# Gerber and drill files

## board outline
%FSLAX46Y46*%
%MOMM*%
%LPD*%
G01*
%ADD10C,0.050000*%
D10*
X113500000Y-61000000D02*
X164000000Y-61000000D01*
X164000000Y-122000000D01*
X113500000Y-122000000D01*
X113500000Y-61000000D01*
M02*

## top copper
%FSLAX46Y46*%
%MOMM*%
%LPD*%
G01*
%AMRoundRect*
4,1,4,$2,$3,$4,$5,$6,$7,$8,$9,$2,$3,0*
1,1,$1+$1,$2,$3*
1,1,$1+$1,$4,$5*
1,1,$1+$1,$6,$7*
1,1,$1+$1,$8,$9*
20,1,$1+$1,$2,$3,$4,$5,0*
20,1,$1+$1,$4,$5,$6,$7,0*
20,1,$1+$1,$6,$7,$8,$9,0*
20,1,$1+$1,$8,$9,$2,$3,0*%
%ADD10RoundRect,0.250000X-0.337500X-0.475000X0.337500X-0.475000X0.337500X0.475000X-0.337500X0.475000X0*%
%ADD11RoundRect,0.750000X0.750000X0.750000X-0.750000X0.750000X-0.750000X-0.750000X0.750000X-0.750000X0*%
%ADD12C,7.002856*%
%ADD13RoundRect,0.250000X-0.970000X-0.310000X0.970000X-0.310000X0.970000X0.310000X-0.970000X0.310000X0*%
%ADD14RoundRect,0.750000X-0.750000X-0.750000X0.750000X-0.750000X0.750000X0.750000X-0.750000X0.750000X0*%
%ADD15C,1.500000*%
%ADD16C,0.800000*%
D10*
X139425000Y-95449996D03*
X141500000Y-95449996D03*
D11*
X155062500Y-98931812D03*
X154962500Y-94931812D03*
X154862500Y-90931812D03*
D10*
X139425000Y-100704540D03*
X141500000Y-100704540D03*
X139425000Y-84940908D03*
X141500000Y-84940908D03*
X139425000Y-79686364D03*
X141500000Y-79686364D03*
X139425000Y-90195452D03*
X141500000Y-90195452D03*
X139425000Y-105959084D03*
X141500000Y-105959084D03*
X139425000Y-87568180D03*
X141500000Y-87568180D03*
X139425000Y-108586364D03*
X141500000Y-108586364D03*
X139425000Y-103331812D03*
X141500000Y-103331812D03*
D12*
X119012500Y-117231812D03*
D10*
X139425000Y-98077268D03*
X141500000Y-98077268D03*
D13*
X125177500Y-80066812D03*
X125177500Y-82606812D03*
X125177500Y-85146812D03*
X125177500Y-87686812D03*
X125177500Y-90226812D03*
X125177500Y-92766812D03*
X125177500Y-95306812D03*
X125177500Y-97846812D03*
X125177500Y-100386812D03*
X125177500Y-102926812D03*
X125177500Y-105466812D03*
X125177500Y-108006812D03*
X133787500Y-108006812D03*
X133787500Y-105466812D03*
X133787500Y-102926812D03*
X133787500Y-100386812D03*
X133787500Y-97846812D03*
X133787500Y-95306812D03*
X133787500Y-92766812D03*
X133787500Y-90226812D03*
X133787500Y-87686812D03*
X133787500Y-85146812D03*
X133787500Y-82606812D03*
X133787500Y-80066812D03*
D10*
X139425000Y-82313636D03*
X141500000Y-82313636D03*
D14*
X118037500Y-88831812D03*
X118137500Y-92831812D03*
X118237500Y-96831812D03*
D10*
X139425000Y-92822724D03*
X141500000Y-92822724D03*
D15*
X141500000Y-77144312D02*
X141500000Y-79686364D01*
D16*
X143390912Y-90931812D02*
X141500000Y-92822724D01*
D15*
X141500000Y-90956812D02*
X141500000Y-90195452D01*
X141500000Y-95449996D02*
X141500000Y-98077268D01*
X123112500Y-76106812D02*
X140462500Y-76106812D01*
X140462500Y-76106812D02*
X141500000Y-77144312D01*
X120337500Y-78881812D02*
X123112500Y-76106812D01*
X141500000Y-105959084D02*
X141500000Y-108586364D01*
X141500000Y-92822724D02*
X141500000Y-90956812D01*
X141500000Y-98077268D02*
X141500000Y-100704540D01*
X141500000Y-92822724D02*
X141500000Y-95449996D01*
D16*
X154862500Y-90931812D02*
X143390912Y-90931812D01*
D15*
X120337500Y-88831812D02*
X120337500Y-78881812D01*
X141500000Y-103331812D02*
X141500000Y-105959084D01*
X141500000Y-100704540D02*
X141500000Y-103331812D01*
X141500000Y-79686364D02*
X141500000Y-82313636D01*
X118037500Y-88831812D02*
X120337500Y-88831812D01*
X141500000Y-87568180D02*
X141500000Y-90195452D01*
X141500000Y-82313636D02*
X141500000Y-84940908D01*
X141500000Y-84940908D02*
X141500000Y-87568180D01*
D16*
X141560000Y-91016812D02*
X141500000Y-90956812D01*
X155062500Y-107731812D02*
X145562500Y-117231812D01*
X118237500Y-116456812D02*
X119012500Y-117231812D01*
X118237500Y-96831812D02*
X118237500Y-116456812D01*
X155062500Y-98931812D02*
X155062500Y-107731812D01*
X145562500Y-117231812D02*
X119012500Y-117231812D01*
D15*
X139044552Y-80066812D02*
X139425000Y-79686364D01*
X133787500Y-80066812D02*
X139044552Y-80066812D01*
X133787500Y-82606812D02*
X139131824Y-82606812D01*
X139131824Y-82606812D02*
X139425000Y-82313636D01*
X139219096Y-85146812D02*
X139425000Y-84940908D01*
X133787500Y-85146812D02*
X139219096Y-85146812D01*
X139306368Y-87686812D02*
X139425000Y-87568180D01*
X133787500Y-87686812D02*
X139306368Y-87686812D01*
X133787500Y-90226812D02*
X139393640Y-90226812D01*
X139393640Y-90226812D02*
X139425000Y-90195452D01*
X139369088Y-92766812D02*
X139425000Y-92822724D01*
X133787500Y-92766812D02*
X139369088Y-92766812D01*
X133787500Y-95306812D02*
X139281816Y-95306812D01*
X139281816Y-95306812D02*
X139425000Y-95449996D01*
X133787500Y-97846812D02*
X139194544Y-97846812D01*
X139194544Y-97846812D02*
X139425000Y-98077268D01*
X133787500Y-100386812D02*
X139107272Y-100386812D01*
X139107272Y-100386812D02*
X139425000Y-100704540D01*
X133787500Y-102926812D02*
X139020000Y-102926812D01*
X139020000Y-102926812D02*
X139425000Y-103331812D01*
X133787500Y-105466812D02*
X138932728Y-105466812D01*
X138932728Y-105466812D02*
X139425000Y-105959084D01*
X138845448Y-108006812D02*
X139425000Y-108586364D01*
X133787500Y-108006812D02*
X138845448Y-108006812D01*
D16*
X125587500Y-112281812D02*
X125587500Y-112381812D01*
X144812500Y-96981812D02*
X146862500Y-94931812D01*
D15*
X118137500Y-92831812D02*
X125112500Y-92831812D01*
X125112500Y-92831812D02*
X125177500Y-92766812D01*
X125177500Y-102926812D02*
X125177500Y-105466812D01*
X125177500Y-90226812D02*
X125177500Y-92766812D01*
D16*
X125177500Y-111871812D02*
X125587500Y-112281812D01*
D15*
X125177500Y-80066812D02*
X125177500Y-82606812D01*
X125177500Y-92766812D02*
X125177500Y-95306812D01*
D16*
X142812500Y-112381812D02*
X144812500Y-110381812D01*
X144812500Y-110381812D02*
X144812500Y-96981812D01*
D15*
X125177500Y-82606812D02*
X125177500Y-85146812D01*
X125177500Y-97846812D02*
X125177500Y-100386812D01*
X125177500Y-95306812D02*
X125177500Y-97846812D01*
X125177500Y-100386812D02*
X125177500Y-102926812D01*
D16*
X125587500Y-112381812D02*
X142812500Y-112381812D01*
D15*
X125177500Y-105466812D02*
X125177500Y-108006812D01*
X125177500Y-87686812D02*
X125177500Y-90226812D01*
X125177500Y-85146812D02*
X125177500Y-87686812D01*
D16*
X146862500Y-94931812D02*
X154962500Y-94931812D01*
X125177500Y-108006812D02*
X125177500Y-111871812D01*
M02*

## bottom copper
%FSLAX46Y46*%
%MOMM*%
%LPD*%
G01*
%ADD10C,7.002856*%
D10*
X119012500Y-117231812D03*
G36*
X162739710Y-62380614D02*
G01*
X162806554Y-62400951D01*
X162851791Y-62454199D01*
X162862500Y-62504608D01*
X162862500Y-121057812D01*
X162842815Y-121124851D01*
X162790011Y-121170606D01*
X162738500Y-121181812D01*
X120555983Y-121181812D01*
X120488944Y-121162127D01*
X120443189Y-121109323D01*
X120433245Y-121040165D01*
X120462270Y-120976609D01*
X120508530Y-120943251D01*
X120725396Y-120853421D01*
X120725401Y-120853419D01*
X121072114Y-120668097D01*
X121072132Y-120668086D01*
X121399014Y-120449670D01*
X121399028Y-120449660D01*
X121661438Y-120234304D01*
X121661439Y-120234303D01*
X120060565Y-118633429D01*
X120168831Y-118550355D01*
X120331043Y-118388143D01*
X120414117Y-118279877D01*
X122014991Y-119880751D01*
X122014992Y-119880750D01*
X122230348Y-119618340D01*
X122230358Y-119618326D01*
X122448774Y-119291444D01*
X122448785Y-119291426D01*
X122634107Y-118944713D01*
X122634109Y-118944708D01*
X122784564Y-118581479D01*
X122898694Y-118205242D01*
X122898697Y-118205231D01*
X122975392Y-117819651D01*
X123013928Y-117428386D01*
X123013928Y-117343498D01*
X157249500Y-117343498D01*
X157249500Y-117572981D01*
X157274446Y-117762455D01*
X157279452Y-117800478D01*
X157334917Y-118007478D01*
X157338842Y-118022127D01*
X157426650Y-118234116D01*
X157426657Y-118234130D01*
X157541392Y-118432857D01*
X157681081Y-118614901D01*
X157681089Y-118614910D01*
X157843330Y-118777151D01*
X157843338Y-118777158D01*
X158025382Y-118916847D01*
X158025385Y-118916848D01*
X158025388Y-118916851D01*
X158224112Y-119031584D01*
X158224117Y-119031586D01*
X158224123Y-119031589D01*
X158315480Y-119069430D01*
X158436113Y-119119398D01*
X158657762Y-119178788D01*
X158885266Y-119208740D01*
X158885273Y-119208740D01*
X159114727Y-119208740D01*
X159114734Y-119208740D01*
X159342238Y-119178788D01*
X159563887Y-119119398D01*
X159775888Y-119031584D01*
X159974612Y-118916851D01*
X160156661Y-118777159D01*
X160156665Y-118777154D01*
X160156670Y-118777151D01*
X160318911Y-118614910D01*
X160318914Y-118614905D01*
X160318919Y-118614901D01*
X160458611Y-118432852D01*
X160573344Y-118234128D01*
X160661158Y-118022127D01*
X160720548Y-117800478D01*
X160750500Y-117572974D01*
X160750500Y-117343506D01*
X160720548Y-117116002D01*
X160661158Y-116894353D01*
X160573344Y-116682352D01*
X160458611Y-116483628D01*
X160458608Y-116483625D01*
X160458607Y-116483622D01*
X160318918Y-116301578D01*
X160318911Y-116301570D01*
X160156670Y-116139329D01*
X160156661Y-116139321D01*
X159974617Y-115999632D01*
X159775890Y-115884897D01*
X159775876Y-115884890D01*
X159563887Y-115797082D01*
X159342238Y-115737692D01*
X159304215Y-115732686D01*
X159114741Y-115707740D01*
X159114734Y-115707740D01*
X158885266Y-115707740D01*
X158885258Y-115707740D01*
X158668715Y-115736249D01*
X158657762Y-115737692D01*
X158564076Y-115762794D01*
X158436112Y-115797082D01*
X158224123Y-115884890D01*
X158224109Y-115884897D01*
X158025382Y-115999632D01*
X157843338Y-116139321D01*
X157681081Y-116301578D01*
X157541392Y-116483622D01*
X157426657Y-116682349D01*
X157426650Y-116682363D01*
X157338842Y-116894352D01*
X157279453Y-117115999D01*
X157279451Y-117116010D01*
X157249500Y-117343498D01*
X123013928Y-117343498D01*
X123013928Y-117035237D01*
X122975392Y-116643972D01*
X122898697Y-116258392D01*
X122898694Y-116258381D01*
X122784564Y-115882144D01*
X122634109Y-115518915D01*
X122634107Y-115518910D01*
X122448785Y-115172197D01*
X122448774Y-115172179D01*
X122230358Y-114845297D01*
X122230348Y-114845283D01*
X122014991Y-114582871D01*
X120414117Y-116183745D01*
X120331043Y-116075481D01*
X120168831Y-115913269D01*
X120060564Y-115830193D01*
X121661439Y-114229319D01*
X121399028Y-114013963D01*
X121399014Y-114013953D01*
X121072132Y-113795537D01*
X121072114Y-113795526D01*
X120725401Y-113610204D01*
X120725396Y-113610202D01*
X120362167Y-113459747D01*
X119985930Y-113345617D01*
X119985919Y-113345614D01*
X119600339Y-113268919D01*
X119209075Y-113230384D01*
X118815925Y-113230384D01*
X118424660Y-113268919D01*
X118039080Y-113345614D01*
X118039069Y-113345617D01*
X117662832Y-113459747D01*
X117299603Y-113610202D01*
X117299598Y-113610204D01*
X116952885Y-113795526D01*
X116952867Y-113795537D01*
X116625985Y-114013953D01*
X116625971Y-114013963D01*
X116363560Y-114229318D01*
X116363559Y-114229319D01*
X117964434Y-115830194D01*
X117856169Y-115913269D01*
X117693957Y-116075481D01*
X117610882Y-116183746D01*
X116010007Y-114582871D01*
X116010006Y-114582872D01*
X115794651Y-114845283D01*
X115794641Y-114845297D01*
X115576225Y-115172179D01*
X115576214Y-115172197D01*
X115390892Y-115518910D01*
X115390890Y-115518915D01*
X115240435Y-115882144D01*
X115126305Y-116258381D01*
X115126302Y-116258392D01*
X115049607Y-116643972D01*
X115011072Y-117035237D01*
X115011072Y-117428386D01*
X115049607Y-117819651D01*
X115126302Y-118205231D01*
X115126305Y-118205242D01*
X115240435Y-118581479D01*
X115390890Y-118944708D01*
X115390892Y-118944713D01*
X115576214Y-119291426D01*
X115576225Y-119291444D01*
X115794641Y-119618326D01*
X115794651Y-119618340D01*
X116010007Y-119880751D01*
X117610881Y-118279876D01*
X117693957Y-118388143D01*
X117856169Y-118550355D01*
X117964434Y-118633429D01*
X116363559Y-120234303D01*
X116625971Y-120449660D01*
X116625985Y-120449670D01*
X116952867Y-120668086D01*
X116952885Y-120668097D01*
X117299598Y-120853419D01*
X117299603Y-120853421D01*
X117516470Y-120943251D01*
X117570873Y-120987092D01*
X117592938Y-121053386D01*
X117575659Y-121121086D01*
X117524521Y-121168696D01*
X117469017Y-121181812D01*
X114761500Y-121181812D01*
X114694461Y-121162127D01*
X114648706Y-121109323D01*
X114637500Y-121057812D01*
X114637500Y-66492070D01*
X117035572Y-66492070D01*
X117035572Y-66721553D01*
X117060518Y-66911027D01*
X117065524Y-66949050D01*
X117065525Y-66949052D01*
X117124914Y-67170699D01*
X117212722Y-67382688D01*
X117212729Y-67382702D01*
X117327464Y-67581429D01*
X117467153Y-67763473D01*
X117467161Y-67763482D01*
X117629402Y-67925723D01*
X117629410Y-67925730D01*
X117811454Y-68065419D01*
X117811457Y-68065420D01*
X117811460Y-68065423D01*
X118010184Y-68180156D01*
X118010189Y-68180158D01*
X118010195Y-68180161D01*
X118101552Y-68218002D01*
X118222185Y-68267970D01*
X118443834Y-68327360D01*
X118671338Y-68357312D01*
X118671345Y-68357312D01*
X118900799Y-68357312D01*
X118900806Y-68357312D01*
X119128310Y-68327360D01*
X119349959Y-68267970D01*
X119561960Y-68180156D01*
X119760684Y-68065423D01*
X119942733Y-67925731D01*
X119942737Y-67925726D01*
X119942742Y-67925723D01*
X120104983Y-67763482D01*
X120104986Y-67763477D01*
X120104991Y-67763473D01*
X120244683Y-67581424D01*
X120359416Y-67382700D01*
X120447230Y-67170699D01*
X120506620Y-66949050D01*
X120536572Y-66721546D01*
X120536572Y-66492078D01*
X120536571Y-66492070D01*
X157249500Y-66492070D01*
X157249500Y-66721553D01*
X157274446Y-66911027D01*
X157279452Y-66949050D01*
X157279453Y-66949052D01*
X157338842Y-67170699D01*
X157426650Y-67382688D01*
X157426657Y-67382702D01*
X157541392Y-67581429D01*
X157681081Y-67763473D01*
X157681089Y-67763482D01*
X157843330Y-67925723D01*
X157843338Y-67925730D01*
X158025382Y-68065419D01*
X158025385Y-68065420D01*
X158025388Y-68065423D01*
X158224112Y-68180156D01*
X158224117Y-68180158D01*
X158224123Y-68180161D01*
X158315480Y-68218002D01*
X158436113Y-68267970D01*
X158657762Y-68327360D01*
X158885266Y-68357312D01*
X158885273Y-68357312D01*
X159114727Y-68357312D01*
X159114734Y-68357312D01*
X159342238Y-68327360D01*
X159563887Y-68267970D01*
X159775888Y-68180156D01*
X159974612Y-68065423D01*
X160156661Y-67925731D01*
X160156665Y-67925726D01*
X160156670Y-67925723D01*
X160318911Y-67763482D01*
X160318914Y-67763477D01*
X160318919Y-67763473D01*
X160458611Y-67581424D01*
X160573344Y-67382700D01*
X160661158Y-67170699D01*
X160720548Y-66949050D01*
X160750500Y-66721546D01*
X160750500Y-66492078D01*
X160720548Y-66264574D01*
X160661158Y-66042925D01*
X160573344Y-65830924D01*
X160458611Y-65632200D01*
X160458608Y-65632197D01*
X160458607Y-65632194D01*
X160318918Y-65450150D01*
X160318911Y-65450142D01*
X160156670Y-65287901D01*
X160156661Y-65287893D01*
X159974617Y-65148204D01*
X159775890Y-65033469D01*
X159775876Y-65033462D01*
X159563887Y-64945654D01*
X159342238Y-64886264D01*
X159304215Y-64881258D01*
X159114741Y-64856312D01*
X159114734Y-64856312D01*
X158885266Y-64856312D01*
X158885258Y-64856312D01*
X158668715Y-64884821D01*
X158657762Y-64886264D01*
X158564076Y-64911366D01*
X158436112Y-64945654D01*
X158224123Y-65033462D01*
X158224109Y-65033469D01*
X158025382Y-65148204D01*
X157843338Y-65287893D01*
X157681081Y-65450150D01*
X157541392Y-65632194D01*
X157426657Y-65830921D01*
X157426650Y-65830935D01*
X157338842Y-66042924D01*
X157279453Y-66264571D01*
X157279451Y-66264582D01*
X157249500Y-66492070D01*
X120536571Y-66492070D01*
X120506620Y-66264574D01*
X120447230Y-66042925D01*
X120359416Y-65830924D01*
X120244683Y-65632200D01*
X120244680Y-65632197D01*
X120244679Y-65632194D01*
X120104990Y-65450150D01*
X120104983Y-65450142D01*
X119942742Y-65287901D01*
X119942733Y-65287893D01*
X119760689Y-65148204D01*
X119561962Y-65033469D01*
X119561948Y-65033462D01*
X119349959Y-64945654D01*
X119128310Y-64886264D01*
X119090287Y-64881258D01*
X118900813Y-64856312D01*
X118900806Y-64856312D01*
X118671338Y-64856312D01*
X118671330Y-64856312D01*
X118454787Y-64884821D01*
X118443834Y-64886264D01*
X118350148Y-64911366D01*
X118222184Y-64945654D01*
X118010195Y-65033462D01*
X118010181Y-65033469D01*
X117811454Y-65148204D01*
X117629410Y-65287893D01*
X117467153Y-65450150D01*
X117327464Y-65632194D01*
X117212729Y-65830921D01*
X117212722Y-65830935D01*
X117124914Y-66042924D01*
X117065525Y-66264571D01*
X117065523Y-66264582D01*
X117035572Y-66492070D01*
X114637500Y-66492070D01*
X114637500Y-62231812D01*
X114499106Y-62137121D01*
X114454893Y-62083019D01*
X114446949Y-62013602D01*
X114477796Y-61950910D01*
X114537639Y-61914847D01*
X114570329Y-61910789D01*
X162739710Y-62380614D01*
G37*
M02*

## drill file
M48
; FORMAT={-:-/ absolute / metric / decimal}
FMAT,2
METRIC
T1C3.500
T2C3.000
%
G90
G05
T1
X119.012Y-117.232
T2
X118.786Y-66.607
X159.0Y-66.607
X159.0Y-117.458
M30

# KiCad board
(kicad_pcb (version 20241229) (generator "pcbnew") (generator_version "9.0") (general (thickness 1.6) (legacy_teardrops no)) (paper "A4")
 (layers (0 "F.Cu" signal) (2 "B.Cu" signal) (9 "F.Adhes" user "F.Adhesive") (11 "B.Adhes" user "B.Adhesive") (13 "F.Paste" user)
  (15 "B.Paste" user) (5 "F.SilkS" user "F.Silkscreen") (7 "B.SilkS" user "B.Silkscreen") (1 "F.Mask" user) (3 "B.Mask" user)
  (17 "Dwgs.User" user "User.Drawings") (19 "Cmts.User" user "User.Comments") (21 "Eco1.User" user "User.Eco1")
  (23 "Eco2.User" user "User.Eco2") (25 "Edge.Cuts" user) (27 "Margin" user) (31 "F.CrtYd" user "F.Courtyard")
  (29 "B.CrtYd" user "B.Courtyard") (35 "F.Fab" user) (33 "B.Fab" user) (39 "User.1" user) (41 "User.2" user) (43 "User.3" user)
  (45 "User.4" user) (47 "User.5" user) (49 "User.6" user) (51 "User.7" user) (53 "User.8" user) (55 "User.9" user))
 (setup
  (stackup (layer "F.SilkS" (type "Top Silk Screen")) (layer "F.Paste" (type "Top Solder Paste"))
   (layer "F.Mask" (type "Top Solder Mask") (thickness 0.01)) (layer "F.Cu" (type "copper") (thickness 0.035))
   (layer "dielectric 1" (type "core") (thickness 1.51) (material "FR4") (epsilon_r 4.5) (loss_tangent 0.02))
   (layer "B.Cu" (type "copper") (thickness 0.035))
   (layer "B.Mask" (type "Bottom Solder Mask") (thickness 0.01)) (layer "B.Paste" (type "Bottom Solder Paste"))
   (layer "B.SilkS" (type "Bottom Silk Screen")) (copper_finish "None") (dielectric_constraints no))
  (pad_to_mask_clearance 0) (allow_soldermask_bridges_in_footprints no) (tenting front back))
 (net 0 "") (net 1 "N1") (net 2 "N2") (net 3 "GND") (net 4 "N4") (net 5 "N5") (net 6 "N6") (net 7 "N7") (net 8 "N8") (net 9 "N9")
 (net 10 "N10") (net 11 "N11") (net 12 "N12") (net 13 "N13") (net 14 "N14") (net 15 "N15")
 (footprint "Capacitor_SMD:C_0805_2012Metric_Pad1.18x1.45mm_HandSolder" (layer "F.Cu") (at 140.4625 95.449996)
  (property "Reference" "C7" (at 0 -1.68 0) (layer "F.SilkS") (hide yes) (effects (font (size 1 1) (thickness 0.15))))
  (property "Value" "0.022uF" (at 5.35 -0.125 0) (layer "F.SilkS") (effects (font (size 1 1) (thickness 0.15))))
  (pad "1" smd roundrect (at -1.0375 0) (size 1.175 1.45) (layers "F.Cu" "F.Mask" "F.Paste") (roundrect_rratio 0.212766) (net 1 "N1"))
  (pad "2" smd roundrect (at 1.0375 0) (size 1.175 1.45) (layers "F.Cu" "F.Mask" "F.Paste") (roundrect_rratio 0.212766) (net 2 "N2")))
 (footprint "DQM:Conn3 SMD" (layer "F.Cu") (at 155.0625 95.031812 180)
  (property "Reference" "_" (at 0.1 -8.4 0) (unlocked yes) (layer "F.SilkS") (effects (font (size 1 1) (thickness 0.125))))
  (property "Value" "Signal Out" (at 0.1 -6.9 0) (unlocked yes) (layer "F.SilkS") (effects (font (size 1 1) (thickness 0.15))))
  (pad "1" smd roundrect (at 0 -3.9 180) (size 3 3) (layers "F.Cu" "F.Mask" "F.Paste") (roundrect_rratio 0.25) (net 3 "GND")
   (thermal_bridge_angle 45))
  (pad "2" smd roundrect (at 0.1 0.1 180) (size 3 3) (layers "F.Cu" "F.Mask" "F.Paste") (roundrect_rratio 0.25) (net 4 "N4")
   (thermal_bridge_angle 45))
  (pad "3" smd roundrect (at 0.2 4.1 180) (size 3 3) (layers "F.Cu" "F.Mask" "F.Paste") (roundrect_rratio 0.25) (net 2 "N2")
   (thermal_bridge_angle 45)))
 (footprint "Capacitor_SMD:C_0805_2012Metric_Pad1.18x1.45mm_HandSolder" (layer "F.Cu") (at 140.4625 100.70454)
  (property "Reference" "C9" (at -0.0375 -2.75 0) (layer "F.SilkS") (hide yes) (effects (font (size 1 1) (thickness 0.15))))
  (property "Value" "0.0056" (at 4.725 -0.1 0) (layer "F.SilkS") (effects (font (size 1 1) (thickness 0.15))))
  (pad "1" smd roundrect (at -1.0375 0) (size 1.175 1.45) (layers "F.Cu" "F.Mask" "F.Paste") (roundrect_rratio 0.212766) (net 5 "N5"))
  (pad "2" smd roundrect (at 1.0375 0) (size 1.175 1.45) (layers "F.Cu" "F.Mask" "F.Paste") (roundrect_rratio 0.212766) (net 2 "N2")))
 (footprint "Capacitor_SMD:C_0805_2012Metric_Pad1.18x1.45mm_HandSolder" (layer "F.Cu") (at 140.4625 84.940908)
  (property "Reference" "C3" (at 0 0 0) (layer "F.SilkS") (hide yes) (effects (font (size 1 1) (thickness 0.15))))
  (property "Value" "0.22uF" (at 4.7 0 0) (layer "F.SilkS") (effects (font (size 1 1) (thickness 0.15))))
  (pad "1" smd roundrect (at -1.0375 0) (size 1.175 1.45) (layers "F.Cu" "F.Mask" "F.Paste") (roundrect_rratio 0.212766) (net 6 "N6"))
  (pad "2" smd roundrect (at 1.0375 0) (size 1.175 1.45) (layers "F.Cu" "F.Mask" "F.Paste") (roundrect_rratio 0.212766) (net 2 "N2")))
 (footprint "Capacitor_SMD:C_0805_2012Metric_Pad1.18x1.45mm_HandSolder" (layer "F.Cu") (at 140.4625 79.686364)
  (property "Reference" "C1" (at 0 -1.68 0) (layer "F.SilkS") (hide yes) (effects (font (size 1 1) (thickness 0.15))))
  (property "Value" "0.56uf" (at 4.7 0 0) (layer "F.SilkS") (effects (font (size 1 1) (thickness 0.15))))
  (pad "1" smd roundrect (at -1.0375 0) (size 1.175 1.45) (layers "F.Cu" "F.Mask" "F.Paste") (roundrect_rratio 0.212766) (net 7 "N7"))
  (pad "2" smd roundrect (at 1.0375 0) (size 1.175 1.45) (layers "F.Cu" "F.Mask" "F.Paste") (roundrect_rratio 0.212766) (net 2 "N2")))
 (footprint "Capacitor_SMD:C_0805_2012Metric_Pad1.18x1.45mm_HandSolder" (layer "F.Cu") (at 140.4625 90.195452)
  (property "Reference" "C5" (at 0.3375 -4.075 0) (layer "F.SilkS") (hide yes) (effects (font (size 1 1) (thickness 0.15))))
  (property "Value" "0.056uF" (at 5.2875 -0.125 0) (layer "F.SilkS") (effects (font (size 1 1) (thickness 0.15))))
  (pad "1" smd roundrect (at -1.0375 0) (size 1.175 1.45) (layers "F.Cu" "F.Mask" "F.Paste") (roundrect_rratio 0.212766) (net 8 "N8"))
  (pad "2" smd roundrect (at 1.0375 0) (size 1.175 1.45) (layers "F.Cu" "F.Mask" "F.Paste") (roundrect_rratio 0.212766) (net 2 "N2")))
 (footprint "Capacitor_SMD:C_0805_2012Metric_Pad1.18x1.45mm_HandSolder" (layer "F.Cu") (at 140.4625 105.959084)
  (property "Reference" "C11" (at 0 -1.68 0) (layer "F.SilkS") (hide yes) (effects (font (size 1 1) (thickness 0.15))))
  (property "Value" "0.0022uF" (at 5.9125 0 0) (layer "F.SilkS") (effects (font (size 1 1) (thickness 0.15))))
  (pad "1" smd roundrect (at -1.0375 0) (size 1.175 1.45) (layers "F.Cu" "F.Mask" "F.Paste") (roundrect_rratio 0.212766) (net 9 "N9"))
  (pad "2" smd roundrect (at 1.0375 0) (size 1.175 1.45) (layers "F.Cu" "F.Mask" "F.Paste") (roundrect_rratio 0.212766) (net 2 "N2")))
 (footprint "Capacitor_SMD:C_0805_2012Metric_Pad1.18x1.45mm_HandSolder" (layer "F.Cu") (at 140.4625 87.56818)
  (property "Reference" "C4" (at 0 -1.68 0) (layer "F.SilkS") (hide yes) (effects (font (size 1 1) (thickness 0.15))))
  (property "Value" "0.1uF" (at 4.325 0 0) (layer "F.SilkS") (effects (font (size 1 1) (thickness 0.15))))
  (pad "1" smd roundrect (at -1.0375 0) (size 1.175 1.45) (layers "F.Cu" "F.Mask" "F.Paste") (roundrect_rratio 0.212766) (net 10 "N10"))
  (pad "2" smd roundrect (at 1.0375 0) (size 1.175 1.45) (layers "F.Cu" "F.Mask" "F.Paste") (roundrect_rratio 0.212766) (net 2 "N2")))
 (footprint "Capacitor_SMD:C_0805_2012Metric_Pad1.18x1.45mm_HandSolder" (layer "F.Cu") (at 140.4625 108.586364)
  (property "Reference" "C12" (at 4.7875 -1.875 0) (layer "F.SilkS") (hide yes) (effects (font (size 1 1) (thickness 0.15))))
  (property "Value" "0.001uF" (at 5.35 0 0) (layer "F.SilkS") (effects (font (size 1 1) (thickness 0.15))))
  (pad "1" smd roundrect (at -1.0375 0) (size 1.175 1.45) (layers "F.Cu" "F.Mask" "F.Paste") (roundrect_rratio 0.212766) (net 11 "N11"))
  (pad "2" smd roundrect (at 1.0375 0) (size 1.175 1.45) (layers "F.Cu" "F.Mask" "F.Paste") (roundrect_rratio 0.212766) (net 2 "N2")))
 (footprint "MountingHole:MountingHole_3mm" (layer "F.Cu") (at 118.786072 66.606812)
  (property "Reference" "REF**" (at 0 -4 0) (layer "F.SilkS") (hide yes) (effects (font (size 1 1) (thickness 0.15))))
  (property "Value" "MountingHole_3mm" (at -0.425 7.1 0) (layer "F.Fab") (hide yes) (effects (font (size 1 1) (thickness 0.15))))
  (pad "" np_thru_hole circle (at 0 0) (size 3 3) (drill 3) (layers "*.Cu" "*.Mask")))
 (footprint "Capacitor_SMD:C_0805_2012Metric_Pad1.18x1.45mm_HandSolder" (layer "F.Cu") (at 140.4625 103.331812)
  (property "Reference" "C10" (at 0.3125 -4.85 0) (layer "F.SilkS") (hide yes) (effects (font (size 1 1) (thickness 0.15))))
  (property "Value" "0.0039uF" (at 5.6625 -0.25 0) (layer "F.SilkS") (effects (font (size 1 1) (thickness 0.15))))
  (pad "1" smd roundrect (at -1.0375 0) (size 1.175 1.45) (layers "F.Cu" "F.Mask" "F.Paste") (roundrect_rratio 0.212766) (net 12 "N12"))
  (pad "2" smd roundrect (at 1.0375 0) (size 1.175 1.45) (layers "F.Cu" "F.Mask" "F.Paste") (roundrect_rratio 0.212766) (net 2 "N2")))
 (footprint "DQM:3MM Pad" (layer "F.Cu") (at 119.0125 117.231812)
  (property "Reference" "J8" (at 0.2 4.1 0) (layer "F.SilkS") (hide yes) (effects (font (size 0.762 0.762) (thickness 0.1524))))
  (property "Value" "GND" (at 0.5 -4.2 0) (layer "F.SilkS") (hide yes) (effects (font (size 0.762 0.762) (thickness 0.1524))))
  (pad "1" thru_hole circle (at 0 0) (size 7.002856 7.002856) (drill 3.5) (layers "*.Cu" "*.Mask") (remove_unused_layers no) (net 3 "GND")))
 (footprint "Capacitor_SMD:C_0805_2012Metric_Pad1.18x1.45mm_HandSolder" (layer "F.Cu") (at 140.4625 98.077268)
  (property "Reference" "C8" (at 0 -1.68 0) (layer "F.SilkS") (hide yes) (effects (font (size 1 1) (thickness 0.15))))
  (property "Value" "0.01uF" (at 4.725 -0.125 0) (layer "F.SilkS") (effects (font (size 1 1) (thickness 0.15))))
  (pad "1" smd roundrect (at -1.0375 0) (size 1.175 1.45) (layers "F.Cu" "F.Mask" "F.Paste") (roundrect_rratio 0.212766) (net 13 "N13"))
  (pad "2" smd roundrect (at 1.0375 0) (size 1.175 1.45) (layers "F.Cu" "F.Mask" "F.Paste") (roundrect_rratio 0.212766) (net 2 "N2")))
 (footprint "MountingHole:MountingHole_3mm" (layer "F.Cu") (at 159 117.45824)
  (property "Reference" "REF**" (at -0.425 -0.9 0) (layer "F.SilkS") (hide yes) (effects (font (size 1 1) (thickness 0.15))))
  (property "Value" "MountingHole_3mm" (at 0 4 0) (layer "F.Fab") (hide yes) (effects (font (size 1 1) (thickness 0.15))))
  (pad "" np_thru_hole circle (at 0 0) (size 3 3) (drill 3) (layers "*.Cu" "*.Mask")))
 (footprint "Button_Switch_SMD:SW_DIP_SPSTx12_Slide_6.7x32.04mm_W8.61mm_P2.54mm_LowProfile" (layer "F.Cu") (at 129.4825 94.036812)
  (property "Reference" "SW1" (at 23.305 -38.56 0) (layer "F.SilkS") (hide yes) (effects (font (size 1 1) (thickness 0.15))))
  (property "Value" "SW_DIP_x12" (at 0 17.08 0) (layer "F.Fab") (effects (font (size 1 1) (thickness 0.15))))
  (pad "1" smd roundrect (at -4.305 -13.97) (size 2.44 1.12) (layers "F.Cu" "F.Mask" "F.Paste") (roundrect_rratio 0.223214) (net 4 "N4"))
  (pad "2" smd roundrect (at -4.305 -11.43) (size 2.44 1.12) (layers "F.Cu" "F.Mask" "F.Paste") (roundrect_rratio 0.223214) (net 4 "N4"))
  (pad "3" smd roundrect (at -4.305 -8.89) (size 2.44 1.12) (layers "F.Cu" "F.Mask" "F.Paste") (roundrect_rratio 0.223214) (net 4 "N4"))
  (pad "4" smd roundrect (at -4.305 -6.35) (size 2.44 1.12) (layers "F.Cu" "F.Mask" "F.Paste") (roundrect_rratio 0.223214) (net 4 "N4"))
  (pad "5" smd roundrect (at -4.305 -3.81) (size 2.44 1.12) (layers "F.Cu" "F.Mask" "F.Paste") (roundrect_rratio 0.223214) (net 4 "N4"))
  (pad "6" smd roundrect (at -4.305 -1.27) (size 2.44 1.12) (layers "F.Cu" "F.Mask" "F.Paste") (roundrect_rratio 0.223214) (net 4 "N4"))
  (pad "7" smd roundrect (at -4.305 1.27) (size 2.44 1.12) (layers "F.Cu" "F.Mask" "F.Paste") (roundrect_rratio 0.223214) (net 4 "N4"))
  (pad "8" smd roundrect (at -4.305 3.81) (size 2.44 1.12) (layers "F.Cu" "F.Mask" "F.Paste") (roundrect_rratio 0.223214) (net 4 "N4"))
  (pad "9" smd roundrect (at -4.305 6.35) (size 2.44 1.12) (layers "F.Cu" "F.Mask" "F.Paste") (roundrect_rratio 0.223214) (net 4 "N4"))
  (pad "10" smd roundrect (at -4.305 8.89) (size 2.44 1.12) (layers "F.Cu" "F.Mask" "F.Paste") (roundrect_rratio 0.223214) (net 4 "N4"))
  (pad "11" smd roundrect (at -4.305 11.43) (size 2.44 1.12) (layers "F.Cu" "F.Mask" "F.Paste") (roundrect_rratio 0.223214) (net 4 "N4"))
  (pad "12" smd roundrect (at -4.305 13.97) (size 2.44 1.12) (layers "F.Cu" "F.Mask" "F.Paste") (roundrect_rratio 0.223214) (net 4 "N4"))
  (pad "13" smd roundrect (at 4.305 13.97) (size 2.44 1.12) (layers "F.Cu" "F.Mask" "F.Paste") (roundrect_rratio 0.223214) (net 11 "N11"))
  (pad "14" smd roundrect (at 4.305 11.43) (size 2.44 1.12) (layers "F.Cu" "F.Mask" "F.Paste") (roundrect_rratio 0.223214) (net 9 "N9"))
  (pad "15" smd roundrect (at 4.305 8.89) (size 2.44 1.12) (layers "F.Cu" "F.Mask" "F.Paste") (roundrect_rratio 0.223214) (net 12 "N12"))
  (pad "16" smd roundrect (at 4.305 6.35) (size 2.44 1.12) (layers "F.Cu" "F.Mask" "F.Paste") (roundrect_rratio 0.223214) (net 5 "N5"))
  (pad "17" smd roundrect (at 4.305 3.81) (size 2.44 1.12) (layers "F.Cu" "F.Mask" "F.Paste") (roundrect_rratio 0.223214) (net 13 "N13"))
  (pad "18" smd roundrect (at 4.305 1.27) (size 2.44 1.12) (layers "F.Cu" "F.Mask" "F.Paste") (roundrect_rratio 0.223214) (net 1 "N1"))
  (pad "19" smd roundrect (at 4.305 -1.27) (size 2.44 1.12) (layers "F.Cu" "F.Mask" "F.Paste") (roundrect_rratio 0.223214) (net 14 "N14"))
  (pad "20" smd roundrect (at 4.305 -3.81) (size 2.44 1.12) (layers "F.Cu" "F.Mask" "F.Paste") (roundrect_rratio 0.223214) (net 8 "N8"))
  (pad "21" smd roundrect (at 4.305 -6.35) (size 2.44 1.12) (layers "F.Cu" "F.Mask" "F.Paste") (roundrect_rratio 0.223214) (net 10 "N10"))
  (pad "22" smd roundrect (at 4.305 -8.89) (size 2.44 1.12) (layers "F.Cu" "F.Mask" "F.Paste") (roundrect_rratio 0.223214) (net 6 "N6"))
  (pad "23" smd roundrect (at 4.305 -11.43) (size 2.44 1.12) (layers "F.Cu" "F.Mask" "F.Paste") (roundrect_rratio 0.223214) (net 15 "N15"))
  (pad "24" smd roundrect (at 4.305 -13.97) (size 2.44 1.12) (layers "F.Cu" "F.Mask" "F.Paste") (roundrect_rratio 0.223214) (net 7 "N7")))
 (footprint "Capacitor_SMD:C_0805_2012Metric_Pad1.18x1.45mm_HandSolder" (layer "F.Cu") (at 140.4625 82.313636)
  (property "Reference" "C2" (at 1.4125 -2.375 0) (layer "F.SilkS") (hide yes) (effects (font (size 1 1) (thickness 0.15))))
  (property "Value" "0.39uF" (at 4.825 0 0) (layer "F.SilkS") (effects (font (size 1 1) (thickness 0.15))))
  (pad "1" smd roundrect (at -1.0375 0) (size 1.175 1.45) (layers "F.Cu" "F.Mask" "F.Paste") (roundrect_rratio 0.212766) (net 15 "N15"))
  (pad "2" smd roundrect (at 1.0375 0) (size 1.175 1.45) (layers "F.Cu" "F.Mask" "F.Paste") (roundrect_rratio 0.212766) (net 2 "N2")))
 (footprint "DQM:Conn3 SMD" (layer "F.Cu") (at 118.0375 92.731812)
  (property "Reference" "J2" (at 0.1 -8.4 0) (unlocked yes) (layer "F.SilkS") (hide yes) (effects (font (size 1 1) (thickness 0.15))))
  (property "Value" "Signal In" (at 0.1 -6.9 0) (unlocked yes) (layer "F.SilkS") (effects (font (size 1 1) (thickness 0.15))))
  (pad "1" smd roundrect (at 0 -3.9) (size 3 3) (layers "F.Cu" "F.Mask" "F.Paste") (roundrect_rratio 0.25) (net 2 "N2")
   (thermal_bridge_angle 45))
  (pad "2" smd roundrect (at 0.1 0.1) (size 3 3) (layers "F.Cu" "F.Mask" "F.Paste") (roundrect_rratio 0.25) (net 4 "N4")
   (thermal_bridge_angle 45))
  (pad "3" smd roundrect (at 0.2 4.1) (size 3 3) (layers "F.Cu" "F.Mask" "F.Paste") (roundrect_rratio 0.25) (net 3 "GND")
   (thermal_bridge_angle 45)))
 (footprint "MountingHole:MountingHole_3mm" (layer "F.Cu") (at 159 66.606812)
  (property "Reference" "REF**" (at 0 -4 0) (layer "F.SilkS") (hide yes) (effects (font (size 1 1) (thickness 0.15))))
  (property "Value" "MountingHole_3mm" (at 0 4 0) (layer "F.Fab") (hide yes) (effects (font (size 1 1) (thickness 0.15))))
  (pad "" np_thru_hole circle (at 0 0) (size 3 3) (drill 3) (layers "*.Cu" "*.Mask")))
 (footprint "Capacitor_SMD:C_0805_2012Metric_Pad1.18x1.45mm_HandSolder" (layer "F.Cu") (at 140.4625 92.822724)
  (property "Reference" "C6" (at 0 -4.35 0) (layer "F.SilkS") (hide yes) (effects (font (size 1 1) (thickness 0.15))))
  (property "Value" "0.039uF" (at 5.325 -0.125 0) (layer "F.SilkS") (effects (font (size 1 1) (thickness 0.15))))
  (pad "1" smd roundrect (at -1.0375 0) (size 1.175 1.45) (layers "F.Cu" "F.Mask" "F.Paste") (roundrect_rratio 0.212766) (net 14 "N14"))
  (pad "2" smd roundrect (at 1.0375 0) (size 1.175 1.45) (layers "F.Cu" "F.Mask" "F.Paste") (roundrect_rratio 0.212766) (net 2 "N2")))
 (gr_rect (start 113.5 61) (end 164 122) (stroke (width 0.05) (type default)) (fill no) (layer "Edge.Cuts"))
 (segment (start 141.5 77.144312) (end 141.5 79.686364) (width 1.5) (layer "F.Cu") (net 2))
 (segment (start 143.390912 90.931812) (end 141.5 92.822724) (width 0.8) (layer "F.Cu") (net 2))
 (segment (start 141.5 90.956812) (end 141.5 90.195452) (width 1.5) (layer "F.Cu") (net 2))
 (segment (start 141.5 95.449996) (end 141.5 98.077268) (width 1.5) (layer "F.Cu") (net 2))
 (segment (start 123.1125 76.106812) (end 140.4625 76.106812) (width 1.5) (layer "F.Cu") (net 2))
 (segment (start 140.4625 76.106812) (end 141.5 77.144312) (width 1.5) (layer "F.Cu") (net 2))
 (segment (start 120.3375 78.881812) (end 123.1125 76.106812) (width 1.5) (layer "F.Cu") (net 2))
 (segment (start 141.5 105.959084) (end 141.5 108.586364) (width 1.5) (layer "F.Cu") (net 2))
 (segment (start 141.5 92.822724) (end 141.5 90.956812) (width 1.5) (layer "F.Cu") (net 2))
 (segment (start 141.5 98.077268) (end 141.5 100.70454) (width 1.5) (layer "F.Cu") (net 2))
 (segment (start 141.5 92.822724) (end 141.5 95.449996) (width 1.5) (layer "F.Cu") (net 2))
 (segment (start 154.8625 90.931812) (end 143.390912 90.931812) (width 0.8) (layer "F.Cu") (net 2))
 (segment (start 120.3375 88.831812) (end 120.3375 78.881812) (width 1.5) (layer "F.Cu") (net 2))
 (segment (start 141.5 103.331812) (end 141.5 105.959084) (width 1.5) (layer "F.Cu") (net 2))
 (segment (start 141.5 100.70454) (end 141.5 103.331812) (width 1.5) (layer "F.Cu") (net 2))
 (segment (start 141.5 79.686364) (end 141.5 82.313636) (width 1.5) (layer "F.Cu") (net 2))
 (segment (start 118.0375 88.831812) (end 120.3375 88.831812) (width 1.5) (layer "F.Cu") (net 2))
 (segment (start 141.5 87.56818) (end 141.5 90.195452) (width 1.5) (layer "F.Cu") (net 2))
 (segment (start 141.5 82.313636) (end 141.5 84.940908) (width 1.5) (layer "F.Cu") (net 2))
 (segment (start 141.5 84.940908) (end 141.5 87.56818) (width 1.5) (layer "F.Cu") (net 2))
 (segment (start 141.56 91.016812) (end 141.5 90.956812) (width 0.8) (layer "F.Cu") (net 2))
 (segment (start 155.0625 107.731812) (end 145.5625 117.231812) (width 0.8) (layer "F.Cu") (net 3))
 (segment (start 118.2375 116.456812) (end 119.0125 117.231812) (width 0.8) (layer "F.Cu") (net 3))
 (segment (start 118.2375 96.831812) (end 118.2375 116.456812) (width 0.8) (layer "F.Cu") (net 3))
 (segment (start 155.0625 98.931812) (end 155.0625 107.731812) (width 0.8) (layer "F.Cu") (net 3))
 (segment (start 145.5625 117.231812) (end 119.0125 117.231812) (width 0.8) (layer "F.Cu") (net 3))
 (segment (start 139.044552 80.066812) (end 139.425 79.686364) (width 1.5) (layer "F.Cu") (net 7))
 (segment (start 133.7875 80.066812) (end 139.044552 80.066812) (width 1.5) (layer "F.Cu") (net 7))
 (segment (start 133.7875 82.606812) (end 139.131824 82.606812) (width 1.5) (layer "F.Cu") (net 15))
 (segment (start 139.131824 82.606812) (end 139.425 82.313636) (width 1.5) (layer "F.Cu") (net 15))
 (segment (start 139.219096 85.146812) (end 139.425 84.940908) (width 1.5) (layer "F.Cu") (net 6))
 (segment (start 133.7875 85.146812) (end 139.219096 85.146812) (width 1.5) (layer "F.Cu") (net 6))
 (segment (start 139.306368 87.686812) (end 139.425 87.56818) (width 1.5) (layer "F.Cu") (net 10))
 (segment (start 133.7875 87.686812) (end 139.306368 87.686812) (width 1.5) (layer "F.Cu") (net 10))
 (segment (start 133.7875 90.226812) (end 139.39364 90.226812) (width 1.5) (layer "F.Cu") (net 8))
 (segment (start 139.39364 90.226812) (end 139.425 90.195452) (width 1.5) (layer "F.Cu") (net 8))
 (segment (start 139.369088 92.766812) (end 139.425 92.822724) (width 1.5) (layer "F.Cu") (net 14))
 (segment (start 133.7875 92.766812) (end 139.369088 92.766812) (width 1.5) (layer "F.Cu") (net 14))
 (segment (start 133.7875 95.306812) (end 139.281816 95.306812) (width 1.5) (layer "F.Cu") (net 1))
 (segment (start 139.281816 95.306812) (end 139.425 95.449996) (width 1.5) (layer "F.Cu") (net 1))
 (segment (start 133.7875 97.846812) (end 139.194544 97.846812) (width 1.5) (layer "F.Cu") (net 13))
 (segment (start 139.194544 97.846812) (end 139.425 98.077268) (width 1.5) (layer "F.Cu") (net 13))
 (segment (start 133.7875 100.386812) (end 139.107272 100.386812) (width 1.5) (layer "F.Cu") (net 5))
 (segment (start 139.107272 100.386812) (end 139.425 100.70454) (width 1.5) (layer "F.Cu") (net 5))
 (segment (start 133.7875 102.926812) (end 139.02 102.926812) (width 1.5) (layer "F.Cu") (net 12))
 (segment (start 139.02 102.926812) (end 139.425 103.331812) (width 1.5) (layer "F.Cu") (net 12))
 (segment (start 133.7875 105.466812) (end 138.932728 105.466812) (width 1.5) (layer "F.Cu") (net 9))
 (segment (start 138.932728 105.466812) (end 139.425 105.959084) (width 1.5) (layer "F.Cu") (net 9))
 (segment (start 138.845448 108.006812) (end 139.425 108.586364) (width 1.5) (layer "F.Cu") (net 11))
 (segment (start 133.7875 108.006812) (end 138.845448 108.006812) (width 1.5) (layer "F.Cu") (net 11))
 (segment (start 125.5875 112.281812) (end 125.5875 112.381812) (width 0.8) (layer "F.Cu") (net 4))
 (segment (start 144.8125 96.981812) (end 146.8625 94.931812) (width 0.8) (layer "F.Cu") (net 4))
 (segment (start 118.1375 92.831812) (end 125.1125 92.831812) (width 1.5) (layer "F.Cu") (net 4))
 (segment (start 125.1125 92.831812) (end 125.1775 92.766812) (width 1.5) (layer "F.Cu") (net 4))
 (segment (start 125.1775 102.926812) (end 125.1775 105.466812) (width 1.5) (layer "F.Cu") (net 4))
 (segment (start 125.1775 90.226812) (end 125.1775 92.766812) (width 1.5) (layer "F.Cu") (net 4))
 (segment (start 125.1775 111.871812) (end 125.5875 112.281812) (width 0.8) (layer "F.Cu") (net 4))
 (segment (start 125.1775 80.066812) (end 125.1775 82.606812) (width 1.5) (layer "F.Cu") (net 4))
 (segment (start 125.1775 92.766812) (end 125.1775 95.306812) (width 1.5) (layer "F.Cu") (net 4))
 (segment (start 142.8125 112.381812) (end 144.8125 110.381812) (width 0.8) (layer "F.Cu") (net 4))
 (segment (start 144.8125 110.381812) (end 144.8125 96.981812) (width 0.8) (layer "F.Cu") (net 4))
 (segment (start 125.1775 82.606812) (end 125.1775 85.146812) (width 1.5) (layer "F.Cu") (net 4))
 (segment (start 125.1775 97.846812) (end 125.1775 100.386812) (width 1.5) (layer "F.Cu") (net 4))
 (segment (start 125.1775 95.306812) (end 125.1775 97.846812) (width 1.5) (layer "F.Cu") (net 4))
 (segment (start 125.1775 100.386812) (end 125.1775 102.926812) (width 1.5) (layer "F.Cu") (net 4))
 (segment (start 125.5875 112.381812) (end 142.8125 112.381812) (width 0.8) (layer "F.Cu") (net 4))
 (segment (start 125.1775 105.466812) (end 125.1775 108.006812) (width 1.5) (layer "F.Cu") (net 4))
 (segment (start 125.1775 87.686812) (end 125.1775 90.226812) (width 1.5) (layer "F.Cu") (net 4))
 (segment (start 125.1775 85.146812) (end 125.1775 87.686812) (width 1.5) (layer "F.Cu") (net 4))
 (segment (start 146.8625 94.931812) (end 154.9625 94.931812) (width 0.8) (layer "F.Cu") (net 4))
 (segment (start 125.1775 108.006812) (end 125.1775 111.871812) (width 0.8) (layer "F.Cu") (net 4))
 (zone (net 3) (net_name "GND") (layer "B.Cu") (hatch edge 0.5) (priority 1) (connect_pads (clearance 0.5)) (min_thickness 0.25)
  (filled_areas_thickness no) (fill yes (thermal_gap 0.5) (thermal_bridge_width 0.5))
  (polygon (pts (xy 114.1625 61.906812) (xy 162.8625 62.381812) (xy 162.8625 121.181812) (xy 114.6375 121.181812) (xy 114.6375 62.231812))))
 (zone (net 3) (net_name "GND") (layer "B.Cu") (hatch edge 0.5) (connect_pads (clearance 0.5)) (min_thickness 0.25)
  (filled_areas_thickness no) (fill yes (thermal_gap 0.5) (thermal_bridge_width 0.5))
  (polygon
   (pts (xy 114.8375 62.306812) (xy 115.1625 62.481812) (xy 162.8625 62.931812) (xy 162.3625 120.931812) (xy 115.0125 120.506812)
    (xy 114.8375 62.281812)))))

